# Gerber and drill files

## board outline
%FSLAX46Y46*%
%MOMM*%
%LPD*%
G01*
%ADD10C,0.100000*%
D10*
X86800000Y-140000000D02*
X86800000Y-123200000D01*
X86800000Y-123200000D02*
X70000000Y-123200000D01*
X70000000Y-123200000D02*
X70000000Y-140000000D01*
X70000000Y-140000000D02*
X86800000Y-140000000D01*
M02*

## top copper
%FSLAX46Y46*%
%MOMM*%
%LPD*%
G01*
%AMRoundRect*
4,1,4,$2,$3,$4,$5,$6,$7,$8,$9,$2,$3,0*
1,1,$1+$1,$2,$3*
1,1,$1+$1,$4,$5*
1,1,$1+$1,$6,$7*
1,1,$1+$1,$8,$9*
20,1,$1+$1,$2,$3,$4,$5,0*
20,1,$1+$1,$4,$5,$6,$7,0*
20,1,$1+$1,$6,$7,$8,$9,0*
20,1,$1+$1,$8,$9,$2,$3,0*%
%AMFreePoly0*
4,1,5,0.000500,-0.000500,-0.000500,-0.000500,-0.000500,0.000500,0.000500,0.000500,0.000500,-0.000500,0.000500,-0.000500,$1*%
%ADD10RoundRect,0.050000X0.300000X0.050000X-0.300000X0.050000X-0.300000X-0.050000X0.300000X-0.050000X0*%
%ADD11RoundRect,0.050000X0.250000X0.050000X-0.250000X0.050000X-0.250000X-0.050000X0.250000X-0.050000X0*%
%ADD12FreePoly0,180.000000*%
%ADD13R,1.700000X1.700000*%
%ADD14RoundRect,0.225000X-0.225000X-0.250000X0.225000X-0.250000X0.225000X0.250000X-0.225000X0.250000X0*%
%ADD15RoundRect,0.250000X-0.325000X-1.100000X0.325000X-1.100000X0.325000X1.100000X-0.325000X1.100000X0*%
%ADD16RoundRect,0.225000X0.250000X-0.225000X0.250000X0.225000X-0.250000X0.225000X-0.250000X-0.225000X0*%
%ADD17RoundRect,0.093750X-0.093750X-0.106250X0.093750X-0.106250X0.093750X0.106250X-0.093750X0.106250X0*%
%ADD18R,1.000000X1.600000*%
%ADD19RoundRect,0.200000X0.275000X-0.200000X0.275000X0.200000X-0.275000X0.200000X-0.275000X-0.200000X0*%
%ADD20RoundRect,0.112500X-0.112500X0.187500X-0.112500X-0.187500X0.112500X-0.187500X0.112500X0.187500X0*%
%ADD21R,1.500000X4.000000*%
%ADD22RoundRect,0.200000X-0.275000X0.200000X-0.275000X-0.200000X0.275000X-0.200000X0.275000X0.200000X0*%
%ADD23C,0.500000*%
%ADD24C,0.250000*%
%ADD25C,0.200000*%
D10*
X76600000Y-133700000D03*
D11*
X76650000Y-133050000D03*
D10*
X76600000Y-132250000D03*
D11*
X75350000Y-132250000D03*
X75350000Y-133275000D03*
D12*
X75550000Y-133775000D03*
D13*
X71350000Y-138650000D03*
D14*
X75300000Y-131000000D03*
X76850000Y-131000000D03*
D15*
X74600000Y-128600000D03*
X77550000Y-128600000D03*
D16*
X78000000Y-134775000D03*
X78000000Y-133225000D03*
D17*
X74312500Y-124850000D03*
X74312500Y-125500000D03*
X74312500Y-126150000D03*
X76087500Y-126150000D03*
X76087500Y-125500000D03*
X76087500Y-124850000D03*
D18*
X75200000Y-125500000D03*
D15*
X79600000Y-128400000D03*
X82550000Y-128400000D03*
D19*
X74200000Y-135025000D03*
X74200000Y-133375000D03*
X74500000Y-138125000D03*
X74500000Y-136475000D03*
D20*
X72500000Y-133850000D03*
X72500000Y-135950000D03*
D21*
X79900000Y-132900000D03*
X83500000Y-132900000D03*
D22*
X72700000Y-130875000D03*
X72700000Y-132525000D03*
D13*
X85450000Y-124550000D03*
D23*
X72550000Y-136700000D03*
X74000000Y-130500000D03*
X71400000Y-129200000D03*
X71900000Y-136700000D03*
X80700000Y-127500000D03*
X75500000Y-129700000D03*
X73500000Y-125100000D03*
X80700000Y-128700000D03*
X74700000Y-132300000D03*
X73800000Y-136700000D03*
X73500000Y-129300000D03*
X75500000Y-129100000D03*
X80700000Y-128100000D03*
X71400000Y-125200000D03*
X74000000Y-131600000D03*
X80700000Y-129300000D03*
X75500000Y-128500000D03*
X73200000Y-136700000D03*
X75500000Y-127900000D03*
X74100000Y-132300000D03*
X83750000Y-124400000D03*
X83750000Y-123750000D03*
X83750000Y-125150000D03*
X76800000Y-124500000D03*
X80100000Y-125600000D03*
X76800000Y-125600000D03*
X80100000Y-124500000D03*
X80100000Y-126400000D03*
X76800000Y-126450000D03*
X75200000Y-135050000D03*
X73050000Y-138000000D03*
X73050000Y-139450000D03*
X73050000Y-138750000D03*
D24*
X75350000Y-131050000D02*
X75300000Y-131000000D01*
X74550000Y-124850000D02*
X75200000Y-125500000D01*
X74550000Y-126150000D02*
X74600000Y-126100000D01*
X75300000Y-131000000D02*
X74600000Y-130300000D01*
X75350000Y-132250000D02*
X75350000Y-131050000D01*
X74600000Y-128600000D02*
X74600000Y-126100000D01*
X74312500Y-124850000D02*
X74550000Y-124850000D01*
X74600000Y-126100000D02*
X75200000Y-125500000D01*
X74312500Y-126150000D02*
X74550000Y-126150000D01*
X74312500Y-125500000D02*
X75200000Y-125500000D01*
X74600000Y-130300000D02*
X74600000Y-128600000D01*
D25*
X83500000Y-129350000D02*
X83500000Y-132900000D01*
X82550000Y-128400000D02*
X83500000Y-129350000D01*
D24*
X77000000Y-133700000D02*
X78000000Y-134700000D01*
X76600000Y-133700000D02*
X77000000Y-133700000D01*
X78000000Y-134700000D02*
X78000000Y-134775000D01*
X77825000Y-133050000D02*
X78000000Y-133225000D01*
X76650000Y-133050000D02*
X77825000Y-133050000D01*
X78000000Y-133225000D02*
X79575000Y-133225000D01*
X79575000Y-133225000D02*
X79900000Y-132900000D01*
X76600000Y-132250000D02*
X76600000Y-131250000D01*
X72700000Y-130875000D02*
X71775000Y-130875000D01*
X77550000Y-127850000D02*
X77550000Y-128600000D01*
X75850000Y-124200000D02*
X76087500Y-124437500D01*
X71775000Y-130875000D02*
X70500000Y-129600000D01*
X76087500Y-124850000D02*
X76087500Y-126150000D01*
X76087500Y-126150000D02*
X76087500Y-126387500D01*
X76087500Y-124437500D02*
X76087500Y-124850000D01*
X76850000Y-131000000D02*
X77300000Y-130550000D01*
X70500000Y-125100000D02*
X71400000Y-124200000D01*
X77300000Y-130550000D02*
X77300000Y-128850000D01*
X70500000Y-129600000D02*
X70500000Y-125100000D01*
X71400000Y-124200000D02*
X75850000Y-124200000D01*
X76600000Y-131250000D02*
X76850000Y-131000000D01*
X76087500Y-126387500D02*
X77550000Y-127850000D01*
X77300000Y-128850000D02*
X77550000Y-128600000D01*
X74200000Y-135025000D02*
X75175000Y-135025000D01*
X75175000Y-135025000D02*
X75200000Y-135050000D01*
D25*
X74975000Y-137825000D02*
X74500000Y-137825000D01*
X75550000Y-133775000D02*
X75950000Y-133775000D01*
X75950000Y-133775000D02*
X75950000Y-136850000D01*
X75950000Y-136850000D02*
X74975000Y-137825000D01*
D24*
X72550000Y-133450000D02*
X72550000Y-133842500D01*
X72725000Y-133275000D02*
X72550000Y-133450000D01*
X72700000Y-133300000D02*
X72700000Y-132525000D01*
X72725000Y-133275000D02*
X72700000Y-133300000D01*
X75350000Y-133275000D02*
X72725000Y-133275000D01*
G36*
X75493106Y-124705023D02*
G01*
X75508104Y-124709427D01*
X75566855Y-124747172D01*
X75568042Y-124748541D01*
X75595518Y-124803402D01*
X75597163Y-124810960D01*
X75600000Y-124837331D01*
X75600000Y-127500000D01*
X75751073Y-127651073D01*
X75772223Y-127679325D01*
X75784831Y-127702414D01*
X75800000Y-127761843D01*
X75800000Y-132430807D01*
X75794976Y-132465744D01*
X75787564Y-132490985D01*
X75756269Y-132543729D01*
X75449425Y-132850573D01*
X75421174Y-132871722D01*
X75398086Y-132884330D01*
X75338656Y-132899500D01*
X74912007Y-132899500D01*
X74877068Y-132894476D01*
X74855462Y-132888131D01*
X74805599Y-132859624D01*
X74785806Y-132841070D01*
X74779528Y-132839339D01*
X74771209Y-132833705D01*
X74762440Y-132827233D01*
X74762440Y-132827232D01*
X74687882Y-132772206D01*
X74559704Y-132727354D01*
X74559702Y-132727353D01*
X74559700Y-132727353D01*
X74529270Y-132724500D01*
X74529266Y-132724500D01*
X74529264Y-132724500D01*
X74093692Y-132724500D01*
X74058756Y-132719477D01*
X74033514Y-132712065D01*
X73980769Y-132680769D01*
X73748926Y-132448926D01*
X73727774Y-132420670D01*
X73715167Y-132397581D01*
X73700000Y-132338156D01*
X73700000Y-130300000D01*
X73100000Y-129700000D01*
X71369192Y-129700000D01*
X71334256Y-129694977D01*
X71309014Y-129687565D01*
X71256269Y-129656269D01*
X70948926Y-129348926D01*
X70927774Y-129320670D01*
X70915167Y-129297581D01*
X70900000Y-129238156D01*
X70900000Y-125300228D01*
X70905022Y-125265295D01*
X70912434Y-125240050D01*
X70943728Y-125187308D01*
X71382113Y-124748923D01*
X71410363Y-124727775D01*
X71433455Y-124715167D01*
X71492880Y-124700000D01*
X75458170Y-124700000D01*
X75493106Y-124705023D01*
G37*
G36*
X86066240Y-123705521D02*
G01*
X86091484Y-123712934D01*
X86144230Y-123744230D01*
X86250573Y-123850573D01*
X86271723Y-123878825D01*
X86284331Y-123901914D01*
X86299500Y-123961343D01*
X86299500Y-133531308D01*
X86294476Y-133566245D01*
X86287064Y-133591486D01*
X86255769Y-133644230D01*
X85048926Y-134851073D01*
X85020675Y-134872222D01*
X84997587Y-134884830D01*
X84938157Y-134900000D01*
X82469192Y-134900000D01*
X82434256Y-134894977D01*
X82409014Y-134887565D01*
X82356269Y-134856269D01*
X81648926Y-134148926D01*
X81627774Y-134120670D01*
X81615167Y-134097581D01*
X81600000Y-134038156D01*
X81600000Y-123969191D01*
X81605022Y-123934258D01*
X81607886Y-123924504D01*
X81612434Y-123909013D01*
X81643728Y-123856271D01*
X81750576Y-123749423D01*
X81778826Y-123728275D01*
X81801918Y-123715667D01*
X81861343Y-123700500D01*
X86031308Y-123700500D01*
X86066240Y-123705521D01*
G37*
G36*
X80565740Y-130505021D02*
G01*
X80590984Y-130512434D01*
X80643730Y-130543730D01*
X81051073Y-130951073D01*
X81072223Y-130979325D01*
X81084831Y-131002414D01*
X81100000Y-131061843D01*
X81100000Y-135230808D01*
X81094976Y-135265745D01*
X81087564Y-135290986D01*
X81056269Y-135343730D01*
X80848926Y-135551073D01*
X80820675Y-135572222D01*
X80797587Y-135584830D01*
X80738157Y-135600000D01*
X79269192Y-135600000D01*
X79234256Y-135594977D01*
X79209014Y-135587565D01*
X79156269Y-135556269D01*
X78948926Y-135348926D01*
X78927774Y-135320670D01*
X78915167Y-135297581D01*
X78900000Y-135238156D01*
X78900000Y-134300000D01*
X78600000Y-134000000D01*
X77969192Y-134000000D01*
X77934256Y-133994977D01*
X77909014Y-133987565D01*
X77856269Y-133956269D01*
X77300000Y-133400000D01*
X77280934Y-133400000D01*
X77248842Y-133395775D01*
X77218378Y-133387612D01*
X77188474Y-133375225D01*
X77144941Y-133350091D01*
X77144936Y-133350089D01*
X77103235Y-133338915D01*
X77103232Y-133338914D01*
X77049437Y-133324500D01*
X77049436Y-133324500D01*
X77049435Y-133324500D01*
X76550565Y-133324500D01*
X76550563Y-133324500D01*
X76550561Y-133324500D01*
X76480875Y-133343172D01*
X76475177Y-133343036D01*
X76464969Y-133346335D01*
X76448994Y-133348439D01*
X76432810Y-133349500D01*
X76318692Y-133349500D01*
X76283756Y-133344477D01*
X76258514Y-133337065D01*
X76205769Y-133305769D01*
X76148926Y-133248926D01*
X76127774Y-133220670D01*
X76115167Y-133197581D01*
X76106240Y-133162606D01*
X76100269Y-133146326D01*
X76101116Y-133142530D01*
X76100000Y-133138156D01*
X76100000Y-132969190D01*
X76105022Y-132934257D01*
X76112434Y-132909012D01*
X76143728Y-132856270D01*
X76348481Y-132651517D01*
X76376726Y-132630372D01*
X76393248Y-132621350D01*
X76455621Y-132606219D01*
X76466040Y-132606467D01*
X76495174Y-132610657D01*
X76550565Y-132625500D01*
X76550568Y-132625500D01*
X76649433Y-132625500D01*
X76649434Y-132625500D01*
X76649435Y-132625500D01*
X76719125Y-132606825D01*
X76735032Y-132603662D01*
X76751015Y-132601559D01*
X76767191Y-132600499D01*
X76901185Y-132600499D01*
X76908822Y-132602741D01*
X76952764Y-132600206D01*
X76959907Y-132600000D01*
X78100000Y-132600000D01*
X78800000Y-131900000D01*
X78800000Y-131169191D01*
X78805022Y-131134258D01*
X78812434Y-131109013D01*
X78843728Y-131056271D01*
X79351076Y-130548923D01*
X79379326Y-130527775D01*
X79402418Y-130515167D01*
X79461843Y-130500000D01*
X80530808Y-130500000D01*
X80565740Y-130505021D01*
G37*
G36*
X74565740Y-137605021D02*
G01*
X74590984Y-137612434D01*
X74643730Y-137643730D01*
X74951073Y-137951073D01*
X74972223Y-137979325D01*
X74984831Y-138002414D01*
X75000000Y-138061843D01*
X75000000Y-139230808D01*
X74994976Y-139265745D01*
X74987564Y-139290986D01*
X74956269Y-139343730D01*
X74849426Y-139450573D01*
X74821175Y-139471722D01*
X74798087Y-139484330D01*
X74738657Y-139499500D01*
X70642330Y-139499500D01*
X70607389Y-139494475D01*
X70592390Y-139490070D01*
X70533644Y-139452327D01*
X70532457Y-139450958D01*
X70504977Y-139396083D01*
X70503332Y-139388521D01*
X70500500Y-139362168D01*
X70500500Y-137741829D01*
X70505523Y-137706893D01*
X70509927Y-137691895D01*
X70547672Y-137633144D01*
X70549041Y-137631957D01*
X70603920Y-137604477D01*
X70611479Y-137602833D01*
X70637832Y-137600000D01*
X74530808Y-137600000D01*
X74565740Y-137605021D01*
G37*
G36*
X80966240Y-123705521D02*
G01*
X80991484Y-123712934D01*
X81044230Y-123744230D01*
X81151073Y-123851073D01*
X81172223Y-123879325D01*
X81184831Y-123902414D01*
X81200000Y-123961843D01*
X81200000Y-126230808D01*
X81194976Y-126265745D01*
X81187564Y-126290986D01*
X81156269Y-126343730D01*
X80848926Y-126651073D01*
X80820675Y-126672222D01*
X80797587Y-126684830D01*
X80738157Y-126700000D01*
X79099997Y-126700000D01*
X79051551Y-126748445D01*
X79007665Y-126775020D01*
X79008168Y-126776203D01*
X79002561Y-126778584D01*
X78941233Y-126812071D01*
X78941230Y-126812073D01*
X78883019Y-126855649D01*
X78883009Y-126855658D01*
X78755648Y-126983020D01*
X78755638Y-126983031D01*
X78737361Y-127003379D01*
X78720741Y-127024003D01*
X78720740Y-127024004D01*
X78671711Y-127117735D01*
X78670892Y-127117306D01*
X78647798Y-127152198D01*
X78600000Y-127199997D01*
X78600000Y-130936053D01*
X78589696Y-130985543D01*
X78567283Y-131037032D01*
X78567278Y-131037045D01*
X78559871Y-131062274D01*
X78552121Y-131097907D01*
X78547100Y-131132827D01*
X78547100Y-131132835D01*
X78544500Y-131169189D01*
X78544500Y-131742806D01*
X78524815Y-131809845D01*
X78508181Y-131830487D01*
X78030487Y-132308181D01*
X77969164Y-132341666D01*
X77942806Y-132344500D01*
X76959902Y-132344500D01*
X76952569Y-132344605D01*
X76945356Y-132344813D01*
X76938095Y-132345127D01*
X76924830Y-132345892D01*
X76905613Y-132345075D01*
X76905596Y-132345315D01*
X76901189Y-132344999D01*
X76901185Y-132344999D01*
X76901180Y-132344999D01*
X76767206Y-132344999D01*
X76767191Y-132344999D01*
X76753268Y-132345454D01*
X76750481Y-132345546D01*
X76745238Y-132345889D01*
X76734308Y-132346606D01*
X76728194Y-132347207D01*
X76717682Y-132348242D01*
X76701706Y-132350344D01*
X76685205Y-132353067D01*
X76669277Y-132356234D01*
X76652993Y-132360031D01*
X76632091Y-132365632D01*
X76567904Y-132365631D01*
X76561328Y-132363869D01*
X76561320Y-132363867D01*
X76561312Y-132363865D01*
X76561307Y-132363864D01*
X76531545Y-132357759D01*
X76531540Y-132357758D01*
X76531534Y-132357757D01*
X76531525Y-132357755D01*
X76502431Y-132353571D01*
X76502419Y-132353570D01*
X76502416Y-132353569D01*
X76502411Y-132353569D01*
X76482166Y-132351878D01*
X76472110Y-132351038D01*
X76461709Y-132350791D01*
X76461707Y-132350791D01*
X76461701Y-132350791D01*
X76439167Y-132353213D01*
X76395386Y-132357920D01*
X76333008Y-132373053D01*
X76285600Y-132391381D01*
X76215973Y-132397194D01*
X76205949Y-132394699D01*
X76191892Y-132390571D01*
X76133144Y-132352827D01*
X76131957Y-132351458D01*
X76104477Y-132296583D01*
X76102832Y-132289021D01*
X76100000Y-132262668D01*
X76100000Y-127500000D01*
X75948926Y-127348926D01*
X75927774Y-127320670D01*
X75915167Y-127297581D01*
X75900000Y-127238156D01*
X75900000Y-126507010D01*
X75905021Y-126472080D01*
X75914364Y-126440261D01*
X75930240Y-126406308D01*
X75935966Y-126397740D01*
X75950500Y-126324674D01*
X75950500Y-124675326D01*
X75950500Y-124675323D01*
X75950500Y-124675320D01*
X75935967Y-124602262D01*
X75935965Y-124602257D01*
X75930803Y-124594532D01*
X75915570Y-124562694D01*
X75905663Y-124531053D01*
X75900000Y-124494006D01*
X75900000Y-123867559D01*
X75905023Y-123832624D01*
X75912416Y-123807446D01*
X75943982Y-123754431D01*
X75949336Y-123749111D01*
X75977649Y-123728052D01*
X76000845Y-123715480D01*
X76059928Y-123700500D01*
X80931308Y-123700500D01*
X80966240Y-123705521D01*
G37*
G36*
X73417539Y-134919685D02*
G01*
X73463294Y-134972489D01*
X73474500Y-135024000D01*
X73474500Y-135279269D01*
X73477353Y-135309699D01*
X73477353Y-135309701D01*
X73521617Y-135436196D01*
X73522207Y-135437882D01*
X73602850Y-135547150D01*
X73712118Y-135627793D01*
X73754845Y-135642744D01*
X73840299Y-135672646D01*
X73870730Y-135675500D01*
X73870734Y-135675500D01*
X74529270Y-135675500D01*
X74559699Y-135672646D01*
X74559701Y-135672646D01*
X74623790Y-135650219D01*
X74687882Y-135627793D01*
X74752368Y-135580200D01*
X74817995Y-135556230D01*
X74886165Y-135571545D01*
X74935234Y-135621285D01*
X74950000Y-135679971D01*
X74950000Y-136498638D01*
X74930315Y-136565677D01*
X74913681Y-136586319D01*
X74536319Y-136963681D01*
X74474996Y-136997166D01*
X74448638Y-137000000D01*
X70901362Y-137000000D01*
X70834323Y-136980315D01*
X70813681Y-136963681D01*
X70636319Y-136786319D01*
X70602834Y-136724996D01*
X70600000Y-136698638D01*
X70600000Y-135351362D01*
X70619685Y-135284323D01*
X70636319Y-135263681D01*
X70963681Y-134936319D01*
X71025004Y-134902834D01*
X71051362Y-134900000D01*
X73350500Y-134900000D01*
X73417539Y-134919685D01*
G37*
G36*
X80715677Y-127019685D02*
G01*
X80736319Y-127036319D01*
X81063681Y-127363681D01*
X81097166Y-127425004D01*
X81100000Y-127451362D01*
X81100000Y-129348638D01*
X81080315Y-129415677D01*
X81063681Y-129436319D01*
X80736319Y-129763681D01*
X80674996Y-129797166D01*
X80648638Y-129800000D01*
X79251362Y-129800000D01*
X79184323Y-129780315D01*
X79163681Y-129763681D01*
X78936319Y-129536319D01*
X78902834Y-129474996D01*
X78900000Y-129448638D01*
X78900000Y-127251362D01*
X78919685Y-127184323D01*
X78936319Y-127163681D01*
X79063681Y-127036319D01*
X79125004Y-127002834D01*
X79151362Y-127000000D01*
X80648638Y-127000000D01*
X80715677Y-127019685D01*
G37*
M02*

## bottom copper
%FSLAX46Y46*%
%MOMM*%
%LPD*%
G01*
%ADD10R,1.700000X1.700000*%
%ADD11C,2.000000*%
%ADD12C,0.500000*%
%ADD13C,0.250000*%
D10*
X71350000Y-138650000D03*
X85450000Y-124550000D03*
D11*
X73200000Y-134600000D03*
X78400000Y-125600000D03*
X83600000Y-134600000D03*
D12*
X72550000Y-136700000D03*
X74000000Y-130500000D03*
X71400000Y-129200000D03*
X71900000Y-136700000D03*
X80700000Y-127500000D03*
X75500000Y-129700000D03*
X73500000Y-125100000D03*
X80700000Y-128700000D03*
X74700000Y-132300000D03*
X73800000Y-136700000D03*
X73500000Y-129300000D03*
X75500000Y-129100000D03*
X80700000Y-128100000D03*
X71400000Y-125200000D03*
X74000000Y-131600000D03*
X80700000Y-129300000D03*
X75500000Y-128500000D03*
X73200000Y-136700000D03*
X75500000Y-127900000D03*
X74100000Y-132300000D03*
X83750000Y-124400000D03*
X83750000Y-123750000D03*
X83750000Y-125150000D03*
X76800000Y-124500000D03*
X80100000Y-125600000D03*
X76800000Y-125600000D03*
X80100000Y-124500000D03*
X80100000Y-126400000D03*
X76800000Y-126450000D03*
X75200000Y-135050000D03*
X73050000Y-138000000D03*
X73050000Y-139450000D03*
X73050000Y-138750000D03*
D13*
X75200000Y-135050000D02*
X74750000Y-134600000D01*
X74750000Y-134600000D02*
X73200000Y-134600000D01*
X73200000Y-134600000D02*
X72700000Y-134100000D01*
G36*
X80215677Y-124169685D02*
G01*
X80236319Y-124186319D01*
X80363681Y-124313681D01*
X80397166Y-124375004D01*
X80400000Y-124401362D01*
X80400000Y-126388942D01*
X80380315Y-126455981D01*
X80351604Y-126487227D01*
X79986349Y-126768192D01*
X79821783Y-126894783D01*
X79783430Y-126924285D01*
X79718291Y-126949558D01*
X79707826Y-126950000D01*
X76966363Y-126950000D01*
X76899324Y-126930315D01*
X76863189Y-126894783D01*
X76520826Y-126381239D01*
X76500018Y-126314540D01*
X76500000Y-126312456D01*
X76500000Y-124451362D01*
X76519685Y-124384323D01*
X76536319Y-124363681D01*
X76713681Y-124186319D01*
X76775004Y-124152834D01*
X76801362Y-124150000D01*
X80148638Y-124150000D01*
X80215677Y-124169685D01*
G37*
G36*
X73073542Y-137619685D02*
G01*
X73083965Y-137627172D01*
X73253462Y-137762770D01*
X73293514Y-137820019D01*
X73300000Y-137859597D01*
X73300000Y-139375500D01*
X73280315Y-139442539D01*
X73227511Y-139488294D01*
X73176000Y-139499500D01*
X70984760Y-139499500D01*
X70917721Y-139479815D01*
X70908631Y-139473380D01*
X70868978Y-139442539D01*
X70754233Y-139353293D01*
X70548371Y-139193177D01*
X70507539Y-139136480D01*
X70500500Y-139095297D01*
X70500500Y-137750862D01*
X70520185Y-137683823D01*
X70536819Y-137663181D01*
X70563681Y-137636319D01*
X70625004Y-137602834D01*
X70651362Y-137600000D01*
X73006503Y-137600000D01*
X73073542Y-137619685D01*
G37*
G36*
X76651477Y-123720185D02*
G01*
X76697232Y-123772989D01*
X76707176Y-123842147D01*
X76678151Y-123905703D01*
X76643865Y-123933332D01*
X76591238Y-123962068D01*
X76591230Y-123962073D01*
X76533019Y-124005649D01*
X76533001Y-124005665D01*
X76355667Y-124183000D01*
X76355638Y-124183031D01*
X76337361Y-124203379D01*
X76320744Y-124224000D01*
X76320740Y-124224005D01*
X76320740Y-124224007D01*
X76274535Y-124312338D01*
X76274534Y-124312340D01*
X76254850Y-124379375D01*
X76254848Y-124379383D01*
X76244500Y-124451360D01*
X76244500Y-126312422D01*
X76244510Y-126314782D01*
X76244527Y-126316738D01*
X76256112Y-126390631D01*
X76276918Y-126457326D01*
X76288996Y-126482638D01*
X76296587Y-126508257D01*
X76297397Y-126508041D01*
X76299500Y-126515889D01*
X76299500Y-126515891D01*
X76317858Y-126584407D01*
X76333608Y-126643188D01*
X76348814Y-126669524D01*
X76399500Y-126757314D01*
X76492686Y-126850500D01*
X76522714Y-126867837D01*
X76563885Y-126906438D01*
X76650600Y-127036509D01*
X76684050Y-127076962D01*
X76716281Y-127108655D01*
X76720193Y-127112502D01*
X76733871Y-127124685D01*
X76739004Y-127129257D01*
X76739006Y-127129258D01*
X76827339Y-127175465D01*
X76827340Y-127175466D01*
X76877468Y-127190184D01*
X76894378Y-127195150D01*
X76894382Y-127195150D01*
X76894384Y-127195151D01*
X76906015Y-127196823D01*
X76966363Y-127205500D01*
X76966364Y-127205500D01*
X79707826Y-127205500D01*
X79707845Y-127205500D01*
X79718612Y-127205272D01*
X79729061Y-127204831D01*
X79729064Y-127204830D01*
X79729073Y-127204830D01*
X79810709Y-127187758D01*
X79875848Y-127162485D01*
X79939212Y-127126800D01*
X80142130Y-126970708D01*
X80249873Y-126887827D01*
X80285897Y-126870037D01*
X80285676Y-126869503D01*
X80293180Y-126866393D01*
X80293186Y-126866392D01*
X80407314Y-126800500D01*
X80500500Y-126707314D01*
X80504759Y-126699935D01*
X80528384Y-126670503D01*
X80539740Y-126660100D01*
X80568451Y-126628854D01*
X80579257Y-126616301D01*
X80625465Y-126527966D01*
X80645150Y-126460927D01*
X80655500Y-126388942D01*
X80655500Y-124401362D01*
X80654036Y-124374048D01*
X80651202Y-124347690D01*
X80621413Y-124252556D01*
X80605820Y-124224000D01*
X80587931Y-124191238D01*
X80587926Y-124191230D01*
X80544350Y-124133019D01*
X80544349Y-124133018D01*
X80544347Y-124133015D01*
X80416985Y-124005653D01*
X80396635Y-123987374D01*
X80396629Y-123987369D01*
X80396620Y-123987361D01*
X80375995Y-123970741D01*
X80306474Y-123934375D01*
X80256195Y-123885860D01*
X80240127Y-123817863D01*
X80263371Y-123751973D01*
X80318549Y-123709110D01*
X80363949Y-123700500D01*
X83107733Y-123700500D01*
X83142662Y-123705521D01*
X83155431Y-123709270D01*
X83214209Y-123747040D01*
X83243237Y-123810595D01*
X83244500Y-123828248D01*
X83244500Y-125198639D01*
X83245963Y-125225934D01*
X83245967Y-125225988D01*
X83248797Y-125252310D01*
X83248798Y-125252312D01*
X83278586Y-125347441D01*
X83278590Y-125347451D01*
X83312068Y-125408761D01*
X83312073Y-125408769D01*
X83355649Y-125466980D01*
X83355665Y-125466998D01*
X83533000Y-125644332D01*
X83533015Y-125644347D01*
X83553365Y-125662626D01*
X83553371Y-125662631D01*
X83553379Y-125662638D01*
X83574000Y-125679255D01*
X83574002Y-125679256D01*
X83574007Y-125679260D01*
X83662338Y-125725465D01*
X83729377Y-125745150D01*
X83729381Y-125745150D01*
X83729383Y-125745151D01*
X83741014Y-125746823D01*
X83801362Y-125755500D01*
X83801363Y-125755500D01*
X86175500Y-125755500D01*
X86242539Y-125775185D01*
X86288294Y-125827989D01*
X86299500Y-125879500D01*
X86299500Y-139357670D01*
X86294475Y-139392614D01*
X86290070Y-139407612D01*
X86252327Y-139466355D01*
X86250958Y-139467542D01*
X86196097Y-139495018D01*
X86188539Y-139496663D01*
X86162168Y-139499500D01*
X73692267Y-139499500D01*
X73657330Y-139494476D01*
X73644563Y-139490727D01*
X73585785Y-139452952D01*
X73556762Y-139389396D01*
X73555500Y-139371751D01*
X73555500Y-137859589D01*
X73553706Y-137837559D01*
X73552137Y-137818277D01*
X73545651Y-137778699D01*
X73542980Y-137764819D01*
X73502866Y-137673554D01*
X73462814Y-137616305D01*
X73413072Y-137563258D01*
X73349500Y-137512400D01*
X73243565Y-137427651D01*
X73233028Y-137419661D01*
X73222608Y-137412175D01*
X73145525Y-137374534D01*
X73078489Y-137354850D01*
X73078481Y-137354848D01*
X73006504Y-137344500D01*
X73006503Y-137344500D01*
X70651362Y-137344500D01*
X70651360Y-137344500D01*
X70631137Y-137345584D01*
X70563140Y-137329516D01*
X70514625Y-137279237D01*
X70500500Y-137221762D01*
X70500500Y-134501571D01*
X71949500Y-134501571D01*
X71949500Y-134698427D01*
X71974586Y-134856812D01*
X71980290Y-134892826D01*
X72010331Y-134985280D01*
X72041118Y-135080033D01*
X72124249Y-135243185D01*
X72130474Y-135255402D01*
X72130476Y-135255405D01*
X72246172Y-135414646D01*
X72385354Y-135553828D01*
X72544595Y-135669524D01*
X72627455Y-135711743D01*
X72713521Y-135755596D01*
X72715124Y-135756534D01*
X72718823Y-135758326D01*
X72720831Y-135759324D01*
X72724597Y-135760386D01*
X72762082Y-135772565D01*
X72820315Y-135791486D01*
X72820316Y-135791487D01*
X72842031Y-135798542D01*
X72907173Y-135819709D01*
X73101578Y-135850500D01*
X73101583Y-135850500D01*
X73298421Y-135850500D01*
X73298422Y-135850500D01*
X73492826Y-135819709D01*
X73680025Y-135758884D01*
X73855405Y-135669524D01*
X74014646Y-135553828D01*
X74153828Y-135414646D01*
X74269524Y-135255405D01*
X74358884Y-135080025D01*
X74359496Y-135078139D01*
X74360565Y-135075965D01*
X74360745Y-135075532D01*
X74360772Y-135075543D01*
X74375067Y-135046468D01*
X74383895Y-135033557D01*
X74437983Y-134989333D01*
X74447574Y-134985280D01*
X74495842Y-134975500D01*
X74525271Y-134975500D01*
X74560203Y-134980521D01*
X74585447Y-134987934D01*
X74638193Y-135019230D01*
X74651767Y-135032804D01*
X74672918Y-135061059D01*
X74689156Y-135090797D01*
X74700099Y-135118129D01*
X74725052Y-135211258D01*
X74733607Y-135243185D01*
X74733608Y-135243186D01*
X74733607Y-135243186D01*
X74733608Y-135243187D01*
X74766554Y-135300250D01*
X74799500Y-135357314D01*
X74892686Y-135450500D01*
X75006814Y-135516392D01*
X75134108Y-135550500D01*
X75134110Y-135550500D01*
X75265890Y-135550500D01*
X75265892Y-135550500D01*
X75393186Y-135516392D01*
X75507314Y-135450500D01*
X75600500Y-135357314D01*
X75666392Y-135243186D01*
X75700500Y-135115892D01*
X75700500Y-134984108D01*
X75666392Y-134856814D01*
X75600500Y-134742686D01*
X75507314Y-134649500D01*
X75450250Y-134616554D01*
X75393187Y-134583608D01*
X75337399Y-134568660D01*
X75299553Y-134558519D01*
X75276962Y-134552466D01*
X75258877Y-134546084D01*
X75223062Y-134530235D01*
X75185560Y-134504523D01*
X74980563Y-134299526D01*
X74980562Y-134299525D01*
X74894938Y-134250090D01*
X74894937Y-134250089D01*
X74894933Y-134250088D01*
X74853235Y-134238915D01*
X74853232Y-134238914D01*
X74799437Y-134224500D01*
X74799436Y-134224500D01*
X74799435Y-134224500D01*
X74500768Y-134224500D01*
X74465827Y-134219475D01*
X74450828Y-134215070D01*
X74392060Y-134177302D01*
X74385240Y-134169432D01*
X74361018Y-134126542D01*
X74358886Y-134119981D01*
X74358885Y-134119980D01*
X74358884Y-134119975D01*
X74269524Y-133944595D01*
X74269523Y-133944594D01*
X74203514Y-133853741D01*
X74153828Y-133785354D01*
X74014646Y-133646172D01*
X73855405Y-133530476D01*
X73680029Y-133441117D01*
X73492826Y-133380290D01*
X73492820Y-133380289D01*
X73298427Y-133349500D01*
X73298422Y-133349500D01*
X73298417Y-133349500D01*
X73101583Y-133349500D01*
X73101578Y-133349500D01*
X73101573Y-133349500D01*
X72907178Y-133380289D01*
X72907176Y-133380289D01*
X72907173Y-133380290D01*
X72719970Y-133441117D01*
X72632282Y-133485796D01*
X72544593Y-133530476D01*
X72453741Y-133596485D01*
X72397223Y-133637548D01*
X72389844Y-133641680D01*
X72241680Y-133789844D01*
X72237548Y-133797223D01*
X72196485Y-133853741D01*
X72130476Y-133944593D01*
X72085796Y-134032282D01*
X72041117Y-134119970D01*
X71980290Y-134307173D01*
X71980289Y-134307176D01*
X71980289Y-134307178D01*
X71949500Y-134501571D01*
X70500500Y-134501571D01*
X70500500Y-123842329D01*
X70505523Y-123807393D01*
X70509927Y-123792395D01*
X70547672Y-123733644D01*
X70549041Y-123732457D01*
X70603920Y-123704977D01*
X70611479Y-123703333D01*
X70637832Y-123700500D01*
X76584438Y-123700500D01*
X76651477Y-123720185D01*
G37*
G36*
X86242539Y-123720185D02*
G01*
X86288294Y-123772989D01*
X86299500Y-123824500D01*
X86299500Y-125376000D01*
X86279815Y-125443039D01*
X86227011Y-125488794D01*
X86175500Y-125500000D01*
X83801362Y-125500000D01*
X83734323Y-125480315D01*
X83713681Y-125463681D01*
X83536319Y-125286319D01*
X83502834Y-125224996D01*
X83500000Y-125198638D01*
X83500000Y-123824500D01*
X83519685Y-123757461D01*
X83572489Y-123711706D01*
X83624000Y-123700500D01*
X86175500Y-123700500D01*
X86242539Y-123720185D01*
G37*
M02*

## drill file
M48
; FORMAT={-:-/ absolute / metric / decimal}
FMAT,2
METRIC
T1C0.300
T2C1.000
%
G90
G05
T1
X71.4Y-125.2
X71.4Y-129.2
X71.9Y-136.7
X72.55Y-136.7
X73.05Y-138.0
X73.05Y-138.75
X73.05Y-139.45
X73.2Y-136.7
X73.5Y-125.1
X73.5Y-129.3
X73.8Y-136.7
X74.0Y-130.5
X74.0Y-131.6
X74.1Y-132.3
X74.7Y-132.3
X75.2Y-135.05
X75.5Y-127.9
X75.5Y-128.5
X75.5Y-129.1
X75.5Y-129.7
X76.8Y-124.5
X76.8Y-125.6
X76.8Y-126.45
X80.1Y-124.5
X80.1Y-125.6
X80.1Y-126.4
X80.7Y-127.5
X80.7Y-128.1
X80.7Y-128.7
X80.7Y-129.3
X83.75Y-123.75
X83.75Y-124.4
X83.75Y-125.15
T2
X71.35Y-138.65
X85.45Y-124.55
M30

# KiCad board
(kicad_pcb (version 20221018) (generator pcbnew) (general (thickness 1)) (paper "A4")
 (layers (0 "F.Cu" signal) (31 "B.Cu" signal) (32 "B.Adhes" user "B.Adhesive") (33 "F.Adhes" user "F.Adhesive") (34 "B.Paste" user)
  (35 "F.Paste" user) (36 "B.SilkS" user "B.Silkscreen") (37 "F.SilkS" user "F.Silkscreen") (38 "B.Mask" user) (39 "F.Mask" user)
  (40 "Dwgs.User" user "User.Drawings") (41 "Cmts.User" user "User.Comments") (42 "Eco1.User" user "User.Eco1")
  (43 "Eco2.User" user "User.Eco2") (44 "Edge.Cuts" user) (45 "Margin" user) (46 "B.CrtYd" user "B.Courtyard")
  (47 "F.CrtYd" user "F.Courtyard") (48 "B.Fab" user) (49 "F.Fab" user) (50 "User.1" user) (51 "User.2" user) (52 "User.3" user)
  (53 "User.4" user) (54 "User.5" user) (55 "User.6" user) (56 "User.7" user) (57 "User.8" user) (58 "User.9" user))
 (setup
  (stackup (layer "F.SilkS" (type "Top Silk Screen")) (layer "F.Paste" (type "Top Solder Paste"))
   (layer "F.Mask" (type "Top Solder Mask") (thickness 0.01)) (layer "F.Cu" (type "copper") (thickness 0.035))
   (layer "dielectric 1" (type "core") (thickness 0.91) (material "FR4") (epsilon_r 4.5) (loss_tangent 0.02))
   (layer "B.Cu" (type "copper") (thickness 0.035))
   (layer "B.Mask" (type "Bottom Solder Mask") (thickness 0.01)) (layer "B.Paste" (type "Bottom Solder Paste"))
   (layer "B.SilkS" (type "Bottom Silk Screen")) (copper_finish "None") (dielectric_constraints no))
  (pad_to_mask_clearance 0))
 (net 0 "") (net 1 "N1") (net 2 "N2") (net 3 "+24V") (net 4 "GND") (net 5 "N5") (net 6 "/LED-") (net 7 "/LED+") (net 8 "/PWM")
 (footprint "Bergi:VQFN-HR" (layer "F.Cu") (at 76 133 180)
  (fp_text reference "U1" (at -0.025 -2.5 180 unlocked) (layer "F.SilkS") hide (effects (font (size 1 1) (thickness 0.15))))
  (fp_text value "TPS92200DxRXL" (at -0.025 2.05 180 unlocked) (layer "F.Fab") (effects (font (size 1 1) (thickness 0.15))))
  (pad "1" smd roundrect (at -0.6 -0.7 180) (size 0.7 0.2) (layers "F.Cu" "F.Mask") (roundrect_rratio 0.25) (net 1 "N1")
   (solder_mask_margin 0.05))
  (pad "2" smd roundrect (at -0.65 -0.05 180) (size 0.6 0.2) (layers "F.Cu" "F.Paste" "F.Mask") (roundrect_rratio 0.25) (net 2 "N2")
   (solder_mask_margin 0.05))
  (pad "3" smd roundrect (at -0.6 0.75 180) (size 0.7 0.2) (layers "F.Cu" "F.Paste" "F.Mask") (roundrect_rratio 0.25) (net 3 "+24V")
   (solder_mask_margin 0.05))
  (pad "4" smd roundrect (at 0.65 0.75 180) (size 0.6 0.2) (layers "F.Cu" "F.Paste" "F.Mask") (roundrect_rratio 0.25) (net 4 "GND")
   (solder_mask_margin 0.05))
  (pad "5" smd roundrect (at 0.65 -0.275 180) (size 0.6 0.2) (layers "F.Cu" "F.Paste" "F.Mask") (roundrect_rratio 0.25) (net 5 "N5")
   (solder_mask_margin 0.05))
  (pad "6" smd custom (at 0.45 -0.775 180) (size 0.001 0.001) (layers "F.Cu" "F.Mask") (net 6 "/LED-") (solder_mask_margin 0.05)
   (options (clearance outline) (anchor rect)) (primitives)))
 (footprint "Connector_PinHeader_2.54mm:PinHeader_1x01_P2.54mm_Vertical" (layer "F.Cu") (at 71.35 138.65)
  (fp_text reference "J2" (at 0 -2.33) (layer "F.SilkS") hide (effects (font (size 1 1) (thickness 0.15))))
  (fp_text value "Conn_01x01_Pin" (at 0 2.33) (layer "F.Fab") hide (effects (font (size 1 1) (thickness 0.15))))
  (pad "1" thru_hole rect (at 0 0) (size 1.7 1.7) (drill 1) (layers "*.Cu" "*.Mask") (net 6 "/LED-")))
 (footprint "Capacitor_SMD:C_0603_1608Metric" (layer "F.Cu") (at 76.075 131)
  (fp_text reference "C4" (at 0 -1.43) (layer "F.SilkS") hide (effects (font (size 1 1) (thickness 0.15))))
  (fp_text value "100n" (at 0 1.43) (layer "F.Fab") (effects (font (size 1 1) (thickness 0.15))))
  (pad "1" smd roundrect (at -0.775 0) (size 0.9 0.95) (layers "F.Cu" "F.Paste" "F.Mask") (roundrect_rratio 0.25) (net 4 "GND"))
  (pad "2" smd roundrect (at 0.775 0) (size 0.9 0.95) (layers "F.Cu" "F.Paste" "F.Mask") (roundrect_rratio 0.25) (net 3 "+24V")))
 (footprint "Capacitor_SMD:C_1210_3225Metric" (layer "F.Cu") (at 76.075 128.6)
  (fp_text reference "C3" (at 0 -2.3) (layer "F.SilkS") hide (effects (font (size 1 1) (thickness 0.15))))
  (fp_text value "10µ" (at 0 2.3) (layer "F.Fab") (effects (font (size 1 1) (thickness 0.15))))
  (pad "1" smd roundrect (at -1.475 0) (size 1.15 2.7) (layers "F.Cu" "F.Paste" "F.Mask") (roundrect_rratio 0.217391) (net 4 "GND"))
  (pad "2" smd roundrect (at 1.475 0) (size 1.15 2.7) (layers "F.Cu" "F.Paste" "F.Mask") (roundrect_rratio 0.217391) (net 3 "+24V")))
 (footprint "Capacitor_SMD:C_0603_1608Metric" (layer "F.Cu") (at 78 134 90)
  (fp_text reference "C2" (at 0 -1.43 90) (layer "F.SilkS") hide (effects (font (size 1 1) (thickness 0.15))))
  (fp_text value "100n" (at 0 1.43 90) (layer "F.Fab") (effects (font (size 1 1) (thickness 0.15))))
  (pad "1" smd roundrect (at -0.775 0 90) (size 0.9 0.95) (layers "F.Cu" "F.Paste" "F.Mask") (roundrect_rratio 0.25) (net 1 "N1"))
  (pad "2" smd roundrect (at 0.775 0 90) (size 0.9 0.95) (layers "F.Cu" "F.Paste" "F.Mask") (roundrect_rratio 0.25) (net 2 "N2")))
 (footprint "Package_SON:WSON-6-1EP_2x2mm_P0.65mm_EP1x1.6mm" (layer "F.Cu") (at 75.2 125.5)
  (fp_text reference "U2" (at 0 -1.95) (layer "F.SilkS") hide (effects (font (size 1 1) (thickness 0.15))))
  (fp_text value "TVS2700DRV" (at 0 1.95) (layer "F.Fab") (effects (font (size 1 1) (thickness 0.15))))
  (pad "" smd roundrect (at 0 -0.4) (size 0.81 0.64) (layers "F.Paste") (roundrect_rratio 0.25))
  (pad "" smd roundrect (at 0 0.4) (size 0.81 0.64) (layers "F.Paste") (roundrect_rratio 0.25))
  (pad "1" smd roundrect (at -0.8875 -0.65) (size 0.375 0.4) (layers "F.Cu" "F.Paste" "F.Mask") (roundrect_rratio 0.25) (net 4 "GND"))
  (pad "2" smd roundrect (at -0.8875 0) (size 0.375 0.4) (layers "F.Cu" "F.Paste" "F.Mask") (roundrect_rratio 0.25) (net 4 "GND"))
  (pad "3" smd roundrect (at -0.8875 0.65) (size 0.375 0.4) (layers "F.Cu" "F.Paste" "F.Mask") (roundrect_rratio 0.25) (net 4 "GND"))
  (pad "4" smd roundrect (at 0.8875 0.65) (size 0.375 0.4) (layers "F.Cu" "F.Paste" "F.Mask") (roundrect_rratio 0.25) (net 3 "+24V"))
  (pad "5" smd roundrect (at 0.8875 0) (size 0.375 0.4) (layers "F.Cu" "F.Paste" "F.Mask") (roundrect_rratio 0.25) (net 3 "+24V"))
  (pad "6" smd roundrect (at 0.8875 -0.65) (size 0.375 0.4) (layers "F.Cu" "F.Paste" "F.Mask") (roundrect_rratio 0.25) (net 3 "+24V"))
  (pad "7" smd rect (at 0 0) (size 1 1.6) (layers "F.Cu" "F.Mask") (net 4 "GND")))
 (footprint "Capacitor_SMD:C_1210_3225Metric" (layer "F.Cu") (at 81.075 128.4)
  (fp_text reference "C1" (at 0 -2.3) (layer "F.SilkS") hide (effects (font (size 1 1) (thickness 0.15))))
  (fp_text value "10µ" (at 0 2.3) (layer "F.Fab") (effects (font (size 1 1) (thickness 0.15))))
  (pad "1" smd roundrect (at -1.475 0) (size 1.15 2.7) (layers "F.Cu" "F.Paste" "F.Mask") (roundrect_rratio 0.217391) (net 4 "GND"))
  (pad "2" smd roundrect (at 1.475 0) (size 1.15 2.7) (layers "F.Cu" "F.Paste" "F.Mask") (roundrect_rratio 0.217391) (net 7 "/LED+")))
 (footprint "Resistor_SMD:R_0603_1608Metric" (layer "F.Cu") (at 74.2 134.2 90)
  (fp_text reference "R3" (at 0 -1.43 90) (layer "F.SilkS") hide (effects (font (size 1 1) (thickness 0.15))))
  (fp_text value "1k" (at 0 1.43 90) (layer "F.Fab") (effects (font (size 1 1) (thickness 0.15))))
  (pad "1" smd roundrect (at -0.825 0 90) (size 0.8 0.95) (layers "F.Cu" "F.Paste" "F.Mask") (roundrect_rratio 0.25) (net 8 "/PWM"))
  (pad "2" smd roundrect (at 0.825 0 90) (size 0.8 0.95) (layers "F.Cu" "F.Paste" "F.Mask") (roundrect_rratio 0.25) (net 5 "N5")))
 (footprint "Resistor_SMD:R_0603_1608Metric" (layer "F.Cu") (at 74.5 137.3 90)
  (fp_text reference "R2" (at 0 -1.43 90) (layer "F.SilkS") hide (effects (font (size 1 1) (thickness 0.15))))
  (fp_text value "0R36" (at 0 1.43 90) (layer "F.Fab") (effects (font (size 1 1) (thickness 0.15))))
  (pad "1" smd roundrect (at -0.825 0 90) (size 0.8 0.95) (layers "F.Cu" "F.Paste" "F.Mask") (roundrect_rratio 0.25) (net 6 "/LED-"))
  (pad "2" smd roundrect (at 0.825 0 90) (size 0.8 0.95) (layers "F.Cu" "F.Paste" "F.Mask") (roundrect_rratio 0.25) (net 4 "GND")))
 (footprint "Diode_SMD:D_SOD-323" (layer "F.Cu") (at 72.5 134.9 -90)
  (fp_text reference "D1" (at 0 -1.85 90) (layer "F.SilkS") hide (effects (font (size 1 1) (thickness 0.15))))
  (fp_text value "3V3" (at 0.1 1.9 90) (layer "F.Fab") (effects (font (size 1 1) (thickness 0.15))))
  (pad "1" smd roundrect (at -1.05 0 270) (size 0.6 0.45) (layers "F.Cu" "F.Paste" "F.Mask") (roundrect_rratio 0.25) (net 5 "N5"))
  (pad "2" smd roundrect (at 1.05 0 270) (size 0.6 0.45) (layers "F.Cu" "F.Paste" "F.Mask") (roundrect_rratio 0.25) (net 4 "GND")))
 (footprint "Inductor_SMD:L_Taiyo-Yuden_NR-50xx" (layer "F.Cu") (at 81.7 132.9)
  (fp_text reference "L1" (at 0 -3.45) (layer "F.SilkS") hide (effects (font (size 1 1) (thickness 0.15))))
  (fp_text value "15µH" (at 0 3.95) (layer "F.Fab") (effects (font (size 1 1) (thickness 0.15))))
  (pad "1" smd rect (at -1.8 0) (size 1.5 4) (layers "F.Cu" "F.Paste" "F.Mask") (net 2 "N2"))
  (pad "2" smd rect (at 1.8 0) (size 1.5 4) (layers "F.Cu" "F.Paste" "F.Mask") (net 7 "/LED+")))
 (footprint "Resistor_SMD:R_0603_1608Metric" (layer "F.Cu") (at 72.7 131.7 -90)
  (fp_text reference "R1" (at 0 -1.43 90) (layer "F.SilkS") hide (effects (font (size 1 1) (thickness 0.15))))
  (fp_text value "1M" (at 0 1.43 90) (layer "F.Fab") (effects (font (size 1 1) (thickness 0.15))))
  (pad "1" smd roundrect (at -0.825 0 270) (size 0.8 0.95) (layers "F.Cu" "F.Paste" "F.Mask") (roundrect_rratio 0.25) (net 3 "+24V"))
  (pad "2" smd roundrect (at 0.825 0 270) (size 0.8 0.95) (layers "F.Cu" "F.Paste" "F.Mask") (roundrect_rratio 0.25) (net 5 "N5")))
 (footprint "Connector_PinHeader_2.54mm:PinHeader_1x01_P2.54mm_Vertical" (layer "F.Cu") (at 85.45 124.55)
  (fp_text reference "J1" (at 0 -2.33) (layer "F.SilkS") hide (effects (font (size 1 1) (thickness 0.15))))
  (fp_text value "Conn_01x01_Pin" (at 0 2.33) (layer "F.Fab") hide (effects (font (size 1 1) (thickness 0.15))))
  (pad "1" thru_hole rect (at 0 0) (size 1.7 1.7) (drill 1) (layers "*.Cu" "*.Mask") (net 7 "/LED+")))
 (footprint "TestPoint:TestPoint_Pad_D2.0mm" (layer "B.Cu") (at 73.2 134.6 180)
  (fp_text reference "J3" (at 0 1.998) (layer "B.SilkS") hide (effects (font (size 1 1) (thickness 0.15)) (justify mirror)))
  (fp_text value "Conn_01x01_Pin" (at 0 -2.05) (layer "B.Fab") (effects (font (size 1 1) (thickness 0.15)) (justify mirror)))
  (pad "1" smd circle (at 0 0 180) (size 2 2) (layers "B.Cu" "B.Mask") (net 8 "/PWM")))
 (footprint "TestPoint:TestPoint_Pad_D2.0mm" (layer "B.Cu") (at 78.4 125.6 180)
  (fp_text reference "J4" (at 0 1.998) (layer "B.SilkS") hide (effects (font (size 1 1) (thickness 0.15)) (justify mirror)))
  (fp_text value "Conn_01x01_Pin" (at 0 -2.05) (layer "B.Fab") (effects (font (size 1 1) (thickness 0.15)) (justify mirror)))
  (pad "1" smd circle (at 0 0 180) (size 2 2) (layers "B.Cu" "B.Mask") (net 3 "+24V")))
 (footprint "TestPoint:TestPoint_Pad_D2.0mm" (layer "B.Cu") (at 83.6 134.6 180)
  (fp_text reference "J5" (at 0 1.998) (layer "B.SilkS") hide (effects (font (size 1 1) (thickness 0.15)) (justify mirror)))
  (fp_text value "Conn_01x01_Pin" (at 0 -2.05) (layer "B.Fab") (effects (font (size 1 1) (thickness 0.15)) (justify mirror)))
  (pad "1" smd circle (at 0 0 180) (size 2 2) (layers "B.Cu" "B.Mask") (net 4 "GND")))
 (gr_line (start 86.8 140) (end 86.8 123.2) (stroke (width 0.1) (type default)) (layer "Edge.Cuts"))
 (gr_line (start 86.8 123.2) (end 70 123.2) (stroke (width 0.1) (type default)) (layer "Edge.Cuts"))
 (gr_line (start 70 123.2) (end 70 140) (stroke (width 0.1) (type default)) (layer "Edge.Cuts"))
 (gr_line (start 70 140) (end 86.8 140) (stroke (width 0.1) (type default)) (layer "Edge.Cuts"))
 (segment (start 75.35 131.05) (end 75.3 131) (width 0.25) (layer "F.Cu") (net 4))
 (segment (start 74.55 124.85) (end 75.2 125.5) (width 0.25) (layer "F.Cu") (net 4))
 (segment (start 74.55 126.15) (end 74.6 126.1) (width 0.25) (layer "F.Cu") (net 4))
 (segment (start 75.3 131) (end 74.6 130.3) (width 0.25) (layer "F.Cu") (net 4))
 (segment (start 75.35 132.25) (end 75.35 131.05) (width 0.25) (layer "F.Cu") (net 4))
 (segment (start 74.6 128.6) (end 74.6 126.1) (width 0.25) (layer "F.Cu") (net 4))
 (segment (start 74.3125 124.85) (end 74.55 124.85) (width 0.25) (layer "F.Cu") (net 4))
 (segment (start 74.6 126.1) (end 75.2 125.5) (width 0.25) (layer "F.Cu") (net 4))
 (segment (start 74.3125 126.15) (end 74.55 126.15) (width 0.25) (layer "F.Cu") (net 4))
 (segment (start 74.3125 125.5) (end 75.2 125.5) (width 0.25) (layer "F.Cu") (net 4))
 (segment (start 74.6 130.3) (end 74.6 128.6) (width 0.25) (layer "F.Cu") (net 4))
 (via (at 72.55 136.7) (size 0.5) (drill 0.3) (layers "F.Cu" "B.Cu") (free) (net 4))
 (via (at 74 130.5) (size 0.5) (drill 0.3) (layers "F.Cu" "B.Cu") (free) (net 4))
 (via (at 71.4 129.2) (size 0.5) (drill 0.3) (layers "F.Cu" "B.Cu") (free) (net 4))
 (via (at 71.9 136.7) (size 0.5) (drill 0.3) (layers "F.Cu" "B.Cu") (free) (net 4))
 (via (at 80.7 127.5) (size 0.5) (drill 0.3) (layers "F.Cu" "B.Cu") (free) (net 4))
 (via (at 75.5 129.7) (size 0.5) (drill 0.3) (layers "F.Cu" "B.Cu") (free) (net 4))
 (via (at 73.5 125.1) (size 0.5) (drill 0.3) (layers "F.Cu" "B.Cu") (free) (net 4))
 (via (at 80.7 128.7) (size 0.5) (drill 0.3) (layers "F.Cu" "B.Cu") (free) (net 4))
 (via (at 74.7 132.3) (size 0.5) (drill 0.3) (layers "F.Cu" "B.Cu") (free) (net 4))
 (via (at 73.8 136.7) (size 0.5) (drill 0.3) (layers "F.Cu" "B.Cu") (free) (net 4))
 (via (at 73.5 129.3) (size 0.5) (drill 0.3) (layers "F.Cu" "B.Cu") (free) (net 4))
 (via (at 75.5 129.1) (size 0.5) (drill 0.3) (layers "F.Cu" "B.Cu") (free) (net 4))
 (via (at 80.7 128.1) (size 0.5) (drill 0.3) (layers "F.Cu" "B.Cu") (free) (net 4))
 (via (at 71.4 125.2) (size 0.5) (drill 0.3) (layers "F.Cu" "B.Cu") (free) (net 4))
 (via (at 74 131.6) (size 0.5) (drill 0.3) (layers "F.Cu" "B.Cu") (free) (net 4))
 (via (at 80.7 129.3) (size 0.5) (drill 0.3) (layers "F.Cu" "B.Cu") (free) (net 4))
 (via (at 75.5 128.5) (size 0.5) (drill 0.3) (layers "F.Cu" "B.Cu") (free) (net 4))
 (via (at 73.2 136.7) (size 0.5) (drill 0.3) (layers "F.Cu" "B.Cu") (free) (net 4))
 (via (at 75.5 127.9) (size 0.5) (drill 0.3) (layers "F.Cu" "B.Cu") (free) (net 4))
 (via (at 74.1 132.3) (size 0.5) (drill 0.3) (layers "F.Cu" "B.Cu") (free) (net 4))
 (segment (start 83.5 129.35) (end 83.5 132.9) (width 0.2) (layer "F.Cu") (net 7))
 (segment (start 82.55 128.4) (end 83.5 129.35) (width 0.2) (layer "F.Cu") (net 7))
 (via (at 83.75 124.4) (size 0.5) (drill 0.3) (layers "F.Cu" "B.Cu") (free) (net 7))
 (via (at 83.75 123.75) (size 0.5) (drill 0.3) (layers "F.Cu" "B.Cu") (free) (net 7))
 (via (at 83.75 125.15) (size 0.5) (drill 0.3) (layers "F.Cu" "B.Cu") (free) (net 7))
 (segment (start 77 133.7) (end 78 134.7) (width 0.25) (layer "F.Cu") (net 1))
 (segment (start 76.6 133.7) (end 77 133.7) (width 0.25) (layer "F.Cu") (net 1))
 (segment (start 78 134.7) (end 78 134.775) (width 0.25) (layer "F.Cu") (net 1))
 (segment (start 77.825 133.05) (end 78 133.225) (width 0.25) (layer "F.Cu") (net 2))
 (segment (start 76.65 133.05) (end 77.825 133.05) (width 0.25) (layer "F.Cu") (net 2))
 (segment (start 78 133.225) (end 79.575 133.225) (width 0.25) (layer "F.Cu") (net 2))
 (segment (start 79.575 133.225) (end 79.9 132.9) (width 0.25) (layer "F.Cu") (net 2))
 (segment (start 76.6 132.25) (end 76.6 131.25) (width 0.25) (layer "F.Cu") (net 3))
 (segment (start 72.7 130.875) (end 71.775 130.875) (width 0.25) (layer "F.Cu") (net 3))
 (segment (start 77.55 127.85) (end 77.55 128.6) (width 0.25) (layer "F.Cu") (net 3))
 (segment (start 75.85 124.2) (end 76.0875 124.4375) (width 0.25) (layer "F.Cu") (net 3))
 (segment (start 71.775 130.875) (end 70.5 129.6) (width 0.25) (layer "F.Cu") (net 3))
 (segment (start 76.0875 124.85) (end 76.0875 126.15) (width 0.25) (layer "F.Cu") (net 3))
 (segment (start 76.0875 126.15) (end 76.0875 126.3875) (width 0.25) (layer "F.Cu") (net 3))
 (segment (start 76.0875 124.4375) (end 76.0875 124.85) (width 0.25) (layer "F.Cu") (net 3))
 (segment (start 76.85 131) (end 77.3 130.55) (width 0.25) (layer "F.Cu") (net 3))
 (segment (start 70.5 125.1) (end 71.4 124.2) (width 0.25) (layer "F.Cu") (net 3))
 (segment (start 77.3 130.55) (end 77.3 128.85) (width 0.25) (layer "F.Cu") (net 3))
 (segment (start 70.5 129.6) (end 70.5 125.1) (width 0.25) (layer "F.Cu") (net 3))
 (segment (start 71.4 124.2) (end 75.85 124.2) (width 0.25) (layer "F.Cu") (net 3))
 (segment (start 76.6 131.25) (end 76.85 131) (width 0.25) (layer "F.Cu") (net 3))
 (segment (start 76.0875 126.3875) (end 77.55 127.85) (width 0.25) (layer "F.Cu") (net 3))
 (segment (start 77.3 128.85) (end 77.55 128.6) (width 0.25) (layer "F.Cu") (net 3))
 (via (at 76.8 124.5) (size 0.5) (drill 0.3) (layers "F.Cu" "B.Cu") (free) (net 3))
 (via (at 80.1 125.6) (size 0.5) (drill 0.3) (layers "F.Cu" "B.Cu") (free) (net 3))
 (via (at 76.8 125.6) (size 0.5) (drill 0.3) (layers "F.Cu" "B.Cu") (free) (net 3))
 (via (at 80.1 124.5) (size 0.5) (drill 0.3) (layers "F.Cu" "B.Cu") (free) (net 3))
 (via (at 80.1 126.4) (size 0.5) (drill 0.3) (layers "F.Cu" "B.Cu") (free) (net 3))
 (via (at 76.8 126.45) (size 0.5) (drill 0.3) (layers "F.Cu" "B.Cu") (free) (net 3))
 (segment (start 74.2 135.025) (end 75.175 135.025) (width 0.25) (layer "F.Cu") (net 8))
 (segment (start 75.175 135.025) (end 75.2 135.05) (width 0.25) (layer "F.Cu") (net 8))
 (via (at 75.2 135.05) (size 0.5) (drill 0.3) (layers "F.Cu" "B.Cu") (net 8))
 (segment (start 75.2 135.05) (end 74.75 134.6) (width 0.25) (layer "B.Cu") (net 8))
 (segment (start 74.75 134.6) (end 73.2 134.6) (width 0.25) (layer "B.Cu") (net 8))
 (segment (start 73.2 134.6) (end 72.7 134.1) (width 0.25) (layer "B.Cu") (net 8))
 (segment (start 74.975 137.825) (end 74.5 137.825) (width 0.2) (layer "F.Cu") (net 6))
 (segment (start 75.55 133.775) (end 75.95 133.775) (width 0.2) (layer "F.Cu") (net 6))
 (segment (start 75.95 133.775) (end 75.95 136.85) (width 0.2) (layer "F.Cu") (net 6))
 (segment (start 75.95 136.85) (end 74.975 137.825) (width 0.2) (layer "F.Cu") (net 6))
 (via (at 73.05 138) (size 0.5) (drill 0.3) (layers "F.Cu" "B.Cu") (free) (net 6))
 (via (at 73.05 139.45) (size 0.5) (drill 0.3) (layers "F.Cu" "B.Cu") (free) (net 6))
 (via (at 73.05 138.75) (size 0.5) (drill 0.3) (layers "F.Cu" "B.Cu") (free) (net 6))
 (segment (start 72.55 133.45) (end 72.55 133.8425) (width 0.25) (layer "F.Cu") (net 5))
 (segment (start 72.725 133.275) (end 72.55 133.45) (width 0.25) (layer "F.Cu") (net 5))
 (segment (start 72.7 133.3) (end 72.7 132.525) (width 0.25) (layer "F.Cu") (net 5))
 (segment (start 72.725 133.275) (end 72.7 133.3) (width 0.25) (layer "F.Cu") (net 5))
 (segment (start 75.35 133.275) (end 72.725 133.275) (width 0.25) (layer "F.Cu") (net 5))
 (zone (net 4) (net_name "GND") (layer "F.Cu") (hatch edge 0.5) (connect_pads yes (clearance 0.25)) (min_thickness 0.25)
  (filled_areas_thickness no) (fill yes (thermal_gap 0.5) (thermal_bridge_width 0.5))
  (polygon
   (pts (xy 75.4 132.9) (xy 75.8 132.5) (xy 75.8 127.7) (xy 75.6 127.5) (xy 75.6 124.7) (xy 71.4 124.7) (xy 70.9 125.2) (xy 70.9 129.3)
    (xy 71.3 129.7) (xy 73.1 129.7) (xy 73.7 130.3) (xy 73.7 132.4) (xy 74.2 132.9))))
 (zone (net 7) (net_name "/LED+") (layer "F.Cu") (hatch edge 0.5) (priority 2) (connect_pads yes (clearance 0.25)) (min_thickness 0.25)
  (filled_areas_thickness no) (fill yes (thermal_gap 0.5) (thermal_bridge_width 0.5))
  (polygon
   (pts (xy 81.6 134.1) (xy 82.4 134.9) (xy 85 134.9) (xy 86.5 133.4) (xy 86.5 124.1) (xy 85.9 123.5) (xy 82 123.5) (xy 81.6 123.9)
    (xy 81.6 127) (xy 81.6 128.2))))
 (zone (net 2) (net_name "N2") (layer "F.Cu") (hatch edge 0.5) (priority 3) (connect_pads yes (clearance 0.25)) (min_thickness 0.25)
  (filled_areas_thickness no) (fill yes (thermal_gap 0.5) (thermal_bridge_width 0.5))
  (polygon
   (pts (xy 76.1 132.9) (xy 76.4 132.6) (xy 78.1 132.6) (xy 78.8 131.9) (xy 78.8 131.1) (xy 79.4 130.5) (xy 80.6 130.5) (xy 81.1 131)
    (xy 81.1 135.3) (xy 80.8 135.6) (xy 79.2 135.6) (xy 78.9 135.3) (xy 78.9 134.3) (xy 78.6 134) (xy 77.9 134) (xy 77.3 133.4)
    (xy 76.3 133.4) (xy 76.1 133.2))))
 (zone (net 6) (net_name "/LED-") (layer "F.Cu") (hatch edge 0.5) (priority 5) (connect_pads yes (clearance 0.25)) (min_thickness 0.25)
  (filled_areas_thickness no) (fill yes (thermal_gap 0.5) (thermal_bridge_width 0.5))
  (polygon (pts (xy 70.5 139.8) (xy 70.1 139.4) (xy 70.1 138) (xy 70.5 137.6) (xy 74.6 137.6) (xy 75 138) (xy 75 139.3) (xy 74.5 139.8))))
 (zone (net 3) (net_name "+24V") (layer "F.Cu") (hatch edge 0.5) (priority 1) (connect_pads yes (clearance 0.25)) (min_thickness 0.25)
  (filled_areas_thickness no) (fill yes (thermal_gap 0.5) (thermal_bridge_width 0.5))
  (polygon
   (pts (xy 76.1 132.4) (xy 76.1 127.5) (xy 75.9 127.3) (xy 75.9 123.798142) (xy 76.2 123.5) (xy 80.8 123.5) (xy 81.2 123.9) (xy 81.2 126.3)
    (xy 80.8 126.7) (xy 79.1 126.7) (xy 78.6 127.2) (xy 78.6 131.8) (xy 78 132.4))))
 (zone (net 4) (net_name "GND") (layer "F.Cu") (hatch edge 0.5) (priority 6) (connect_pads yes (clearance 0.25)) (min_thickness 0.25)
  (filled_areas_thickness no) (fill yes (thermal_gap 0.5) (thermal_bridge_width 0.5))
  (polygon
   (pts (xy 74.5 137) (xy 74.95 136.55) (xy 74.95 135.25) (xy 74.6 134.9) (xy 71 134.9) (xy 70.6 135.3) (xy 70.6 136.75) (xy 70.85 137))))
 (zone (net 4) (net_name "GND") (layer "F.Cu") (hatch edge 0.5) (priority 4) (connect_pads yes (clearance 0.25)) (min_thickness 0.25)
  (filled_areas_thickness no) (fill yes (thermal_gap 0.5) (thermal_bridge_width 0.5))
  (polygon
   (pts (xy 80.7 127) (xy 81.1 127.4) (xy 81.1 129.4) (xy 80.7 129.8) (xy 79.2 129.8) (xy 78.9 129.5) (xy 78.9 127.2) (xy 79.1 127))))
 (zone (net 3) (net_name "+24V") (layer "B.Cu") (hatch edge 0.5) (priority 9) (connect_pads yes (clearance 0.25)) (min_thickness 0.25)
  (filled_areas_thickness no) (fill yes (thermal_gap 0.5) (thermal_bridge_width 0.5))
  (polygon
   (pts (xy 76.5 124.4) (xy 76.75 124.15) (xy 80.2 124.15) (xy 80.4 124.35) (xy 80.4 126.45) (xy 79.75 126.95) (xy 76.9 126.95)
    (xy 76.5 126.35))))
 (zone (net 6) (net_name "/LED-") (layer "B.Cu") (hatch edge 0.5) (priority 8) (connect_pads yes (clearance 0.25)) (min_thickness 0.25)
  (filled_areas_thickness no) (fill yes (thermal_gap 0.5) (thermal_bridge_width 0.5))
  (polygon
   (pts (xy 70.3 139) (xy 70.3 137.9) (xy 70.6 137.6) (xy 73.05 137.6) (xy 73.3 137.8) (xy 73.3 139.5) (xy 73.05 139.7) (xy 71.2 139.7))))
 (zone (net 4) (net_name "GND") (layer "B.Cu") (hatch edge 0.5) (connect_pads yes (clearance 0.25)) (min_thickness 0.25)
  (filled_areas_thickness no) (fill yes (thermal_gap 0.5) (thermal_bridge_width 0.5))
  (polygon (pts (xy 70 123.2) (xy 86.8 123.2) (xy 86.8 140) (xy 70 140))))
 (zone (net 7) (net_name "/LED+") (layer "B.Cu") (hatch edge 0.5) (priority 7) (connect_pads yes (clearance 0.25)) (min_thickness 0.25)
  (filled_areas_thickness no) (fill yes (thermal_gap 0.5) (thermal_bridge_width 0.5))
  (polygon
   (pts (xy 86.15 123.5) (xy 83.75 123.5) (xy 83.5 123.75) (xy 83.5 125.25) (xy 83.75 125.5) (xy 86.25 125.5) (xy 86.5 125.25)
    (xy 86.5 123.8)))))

